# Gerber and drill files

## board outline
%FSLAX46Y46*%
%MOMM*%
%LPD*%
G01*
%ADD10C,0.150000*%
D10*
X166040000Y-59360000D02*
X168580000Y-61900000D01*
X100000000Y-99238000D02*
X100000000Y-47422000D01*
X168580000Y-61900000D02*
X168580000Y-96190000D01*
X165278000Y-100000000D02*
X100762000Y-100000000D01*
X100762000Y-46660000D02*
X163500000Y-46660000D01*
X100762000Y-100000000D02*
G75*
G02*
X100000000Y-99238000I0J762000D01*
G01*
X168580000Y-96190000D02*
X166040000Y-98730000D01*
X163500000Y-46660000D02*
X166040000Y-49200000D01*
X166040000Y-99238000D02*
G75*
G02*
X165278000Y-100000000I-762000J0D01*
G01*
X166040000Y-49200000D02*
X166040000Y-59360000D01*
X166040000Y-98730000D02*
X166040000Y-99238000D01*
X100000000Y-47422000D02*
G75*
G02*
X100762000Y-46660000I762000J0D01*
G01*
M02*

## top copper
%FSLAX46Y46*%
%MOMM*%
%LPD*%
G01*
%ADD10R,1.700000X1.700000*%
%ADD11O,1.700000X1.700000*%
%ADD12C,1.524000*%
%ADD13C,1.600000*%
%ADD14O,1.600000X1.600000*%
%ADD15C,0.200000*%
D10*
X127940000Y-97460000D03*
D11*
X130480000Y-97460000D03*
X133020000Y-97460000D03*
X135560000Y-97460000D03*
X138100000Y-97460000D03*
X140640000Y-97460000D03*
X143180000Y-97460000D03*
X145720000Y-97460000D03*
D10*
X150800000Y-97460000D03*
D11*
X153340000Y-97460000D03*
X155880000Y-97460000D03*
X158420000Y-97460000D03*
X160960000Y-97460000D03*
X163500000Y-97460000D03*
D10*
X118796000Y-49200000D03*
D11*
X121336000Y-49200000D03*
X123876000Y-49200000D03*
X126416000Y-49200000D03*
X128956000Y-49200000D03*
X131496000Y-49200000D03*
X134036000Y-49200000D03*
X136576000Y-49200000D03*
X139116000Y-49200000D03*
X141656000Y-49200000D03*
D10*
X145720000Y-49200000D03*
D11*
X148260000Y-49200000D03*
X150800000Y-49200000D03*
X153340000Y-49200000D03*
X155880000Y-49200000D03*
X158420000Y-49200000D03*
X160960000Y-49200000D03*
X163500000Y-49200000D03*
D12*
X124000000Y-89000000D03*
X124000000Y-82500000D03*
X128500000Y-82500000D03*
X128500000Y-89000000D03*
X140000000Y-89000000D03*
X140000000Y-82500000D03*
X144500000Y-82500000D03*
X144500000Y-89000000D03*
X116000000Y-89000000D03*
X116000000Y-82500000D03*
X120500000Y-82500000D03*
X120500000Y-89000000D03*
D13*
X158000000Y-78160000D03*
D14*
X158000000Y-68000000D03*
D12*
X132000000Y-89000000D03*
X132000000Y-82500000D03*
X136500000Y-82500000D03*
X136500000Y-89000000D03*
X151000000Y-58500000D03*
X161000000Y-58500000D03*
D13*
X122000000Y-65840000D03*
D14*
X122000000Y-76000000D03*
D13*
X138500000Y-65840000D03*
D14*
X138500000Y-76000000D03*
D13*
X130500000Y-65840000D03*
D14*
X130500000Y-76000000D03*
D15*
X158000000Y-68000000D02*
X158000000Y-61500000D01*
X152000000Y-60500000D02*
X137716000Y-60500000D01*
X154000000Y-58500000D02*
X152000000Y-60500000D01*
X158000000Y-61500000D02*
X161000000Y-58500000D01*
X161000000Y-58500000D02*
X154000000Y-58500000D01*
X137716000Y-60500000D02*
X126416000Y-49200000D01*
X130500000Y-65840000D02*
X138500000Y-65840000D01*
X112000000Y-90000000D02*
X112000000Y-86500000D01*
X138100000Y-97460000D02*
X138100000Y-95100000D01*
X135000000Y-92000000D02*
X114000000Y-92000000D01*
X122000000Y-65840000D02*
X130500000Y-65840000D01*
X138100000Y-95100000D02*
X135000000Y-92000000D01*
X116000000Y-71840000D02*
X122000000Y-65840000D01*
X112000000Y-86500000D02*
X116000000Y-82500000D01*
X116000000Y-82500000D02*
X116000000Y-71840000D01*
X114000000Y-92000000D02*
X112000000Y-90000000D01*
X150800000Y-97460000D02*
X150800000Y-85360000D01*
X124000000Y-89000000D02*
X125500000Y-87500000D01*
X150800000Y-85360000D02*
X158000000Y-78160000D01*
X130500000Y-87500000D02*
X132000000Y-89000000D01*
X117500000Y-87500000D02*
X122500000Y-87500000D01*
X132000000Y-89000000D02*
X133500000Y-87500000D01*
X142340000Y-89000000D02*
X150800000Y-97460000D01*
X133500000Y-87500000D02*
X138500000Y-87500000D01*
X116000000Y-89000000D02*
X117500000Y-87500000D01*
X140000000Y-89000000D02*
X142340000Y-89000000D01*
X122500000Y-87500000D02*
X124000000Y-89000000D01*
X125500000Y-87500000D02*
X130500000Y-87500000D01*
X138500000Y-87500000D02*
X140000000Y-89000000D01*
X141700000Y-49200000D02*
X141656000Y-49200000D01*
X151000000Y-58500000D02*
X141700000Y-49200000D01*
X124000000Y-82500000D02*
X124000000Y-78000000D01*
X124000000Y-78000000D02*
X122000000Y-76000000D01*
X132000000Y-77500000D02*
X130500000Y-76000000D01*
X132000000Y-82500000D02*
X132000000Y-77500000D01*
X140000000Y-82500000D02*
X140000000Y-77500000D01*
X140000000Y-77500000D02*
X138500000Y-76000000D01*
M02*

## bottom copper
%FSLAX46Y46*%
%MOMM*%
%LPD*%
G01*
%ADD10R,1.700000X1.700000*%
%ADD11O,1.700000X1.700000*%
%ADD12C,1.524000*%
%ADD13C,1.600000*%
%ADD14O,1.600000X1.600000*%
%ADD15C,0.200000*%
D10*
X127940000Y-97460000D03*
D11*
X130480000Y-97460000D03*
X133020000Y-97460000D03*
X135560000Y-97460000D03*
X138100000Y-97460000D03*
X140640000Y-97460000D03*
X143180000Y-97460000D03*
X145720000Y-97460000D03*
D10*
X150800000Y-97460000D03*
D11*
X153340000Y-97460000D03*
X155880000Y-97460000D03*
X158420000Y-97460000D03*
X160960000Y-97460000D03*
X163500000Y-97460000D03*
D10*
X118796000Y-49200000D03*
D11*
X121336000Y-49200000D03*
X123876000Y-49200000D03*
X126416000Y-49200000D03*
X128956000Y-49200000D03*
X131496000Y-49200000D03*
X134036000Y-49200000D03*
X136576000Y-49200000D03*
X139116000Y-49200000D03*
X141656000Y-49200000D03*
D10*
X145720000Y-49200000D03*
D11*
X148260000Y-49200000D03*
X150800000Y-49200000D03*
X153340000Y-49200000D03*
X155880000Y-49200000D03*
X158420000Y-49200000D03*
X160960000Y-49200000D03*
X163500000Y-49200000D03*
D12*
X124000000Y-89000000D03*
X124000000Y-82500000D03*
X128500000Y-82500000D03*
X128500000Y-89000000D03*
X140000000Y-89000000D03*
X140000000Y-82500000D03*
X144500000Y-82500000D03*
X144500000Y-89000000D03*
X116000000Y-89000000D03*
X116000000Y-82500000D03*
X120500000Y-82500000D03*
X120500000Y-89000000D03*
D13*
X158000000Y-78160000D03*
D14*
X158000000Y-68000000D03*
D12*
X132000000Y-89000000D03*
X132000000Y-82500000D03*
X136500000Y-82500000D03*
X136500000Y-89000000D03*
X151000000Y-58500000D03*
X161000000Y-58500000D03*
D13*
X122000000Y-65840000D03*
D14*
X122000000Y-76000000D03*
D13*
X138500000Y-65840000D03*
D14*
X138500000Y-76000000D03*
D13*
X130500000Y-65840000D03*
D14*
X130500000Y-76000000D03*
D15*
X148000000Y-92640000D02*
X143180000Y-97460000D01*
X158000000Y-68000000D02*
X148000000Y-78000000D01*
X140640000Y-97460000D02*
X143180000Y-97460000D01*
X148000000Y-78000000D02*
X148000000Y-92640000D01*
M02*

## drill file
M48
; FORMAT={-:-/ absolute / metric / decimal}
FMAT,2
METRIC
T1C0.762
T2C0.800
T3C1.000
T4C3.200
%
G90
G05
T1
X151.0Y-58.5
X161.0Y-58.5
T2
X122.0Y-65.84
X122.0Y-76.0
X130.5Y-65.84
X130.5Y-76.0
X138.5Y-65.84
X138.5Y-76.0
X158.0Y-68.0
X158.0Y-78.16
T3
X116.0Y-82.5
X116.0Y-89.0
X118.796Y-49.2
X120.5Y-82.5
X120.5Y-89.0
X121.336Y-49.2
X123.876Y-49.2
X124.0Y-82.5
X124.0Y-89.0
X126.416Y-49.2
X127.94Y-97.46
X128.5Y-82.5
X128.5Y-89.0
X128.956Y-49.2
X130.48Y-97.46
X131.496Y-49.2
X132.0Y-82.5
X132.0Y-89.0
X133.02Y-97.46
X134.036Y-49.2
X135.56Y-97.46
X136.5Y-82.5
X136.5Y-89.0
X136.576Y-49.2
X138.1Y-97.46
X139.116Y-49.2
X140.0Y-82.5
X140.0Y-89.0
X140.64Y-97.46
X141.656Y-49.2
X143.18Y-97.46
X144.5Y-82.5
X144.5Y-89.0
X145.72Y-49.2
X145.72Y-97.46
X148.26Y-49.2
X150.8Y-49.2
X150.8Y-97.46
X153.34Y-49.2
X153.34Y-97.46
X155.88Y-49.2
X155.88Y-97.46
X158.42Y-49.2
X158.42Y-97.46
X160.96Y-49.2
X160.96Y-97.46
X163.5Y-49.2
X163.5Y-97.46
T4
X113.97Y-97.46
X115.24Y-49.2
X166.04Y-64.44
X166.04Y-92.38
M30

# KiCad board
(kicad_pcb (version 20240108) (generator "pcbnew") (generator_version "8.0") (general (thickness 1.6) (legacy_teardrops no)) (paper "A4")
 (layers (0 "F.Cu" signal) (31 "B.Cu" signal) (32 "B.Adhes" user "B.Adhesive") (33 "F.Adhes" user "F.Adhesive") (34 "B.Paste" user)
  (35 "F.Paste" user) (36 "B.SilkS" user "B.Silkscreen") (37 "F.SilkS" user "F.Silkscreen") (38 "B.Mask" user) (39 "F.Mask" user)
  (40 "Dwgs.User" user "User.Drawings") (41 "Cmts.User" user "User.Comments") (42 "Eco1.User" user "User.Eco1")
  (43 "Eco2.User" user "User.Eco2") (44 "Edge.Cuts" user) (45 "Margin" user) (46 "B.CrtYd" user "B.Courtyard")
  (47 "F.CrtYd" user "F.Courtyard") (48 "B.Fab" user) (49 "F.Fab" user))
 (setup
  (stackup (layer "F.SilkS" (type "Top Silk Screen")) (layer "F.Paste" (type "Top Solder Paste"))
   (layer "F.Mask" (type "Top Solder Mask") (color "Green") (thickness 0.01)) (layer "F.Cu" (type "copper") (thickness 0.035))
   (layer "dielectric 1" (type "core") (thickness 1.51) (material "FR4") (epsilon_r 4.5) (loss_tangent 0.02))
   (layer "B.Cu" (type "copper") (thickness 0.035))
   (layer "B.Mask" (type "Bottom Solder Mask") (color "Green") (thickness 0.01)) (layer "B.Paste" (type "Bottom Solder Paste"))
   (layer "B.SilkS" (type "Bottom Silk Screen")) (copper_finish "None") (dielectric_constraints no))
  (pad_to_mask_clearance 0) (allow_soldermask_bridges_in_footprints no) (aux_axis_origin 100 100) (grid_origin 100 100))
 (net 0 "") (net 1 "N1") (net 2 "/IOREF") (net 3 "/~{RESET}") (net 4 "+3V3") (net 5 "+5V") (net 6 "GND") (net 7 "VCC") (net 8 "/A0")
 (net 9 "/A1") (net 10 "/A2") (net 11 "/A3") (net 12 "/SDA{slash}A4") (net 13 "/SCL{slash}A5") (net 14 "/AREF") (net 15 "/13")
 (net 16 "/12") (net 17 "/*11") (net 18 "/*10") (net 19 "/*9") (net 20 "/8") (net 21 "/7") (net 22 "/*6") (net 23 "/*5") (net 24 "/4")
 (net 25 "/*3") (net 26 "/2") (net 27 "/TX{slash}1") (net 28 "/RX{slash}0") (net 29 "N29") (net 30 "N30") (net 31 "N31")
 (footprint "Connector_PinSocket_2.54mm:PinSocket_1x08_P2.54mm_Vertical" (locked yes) (layer "F.Cu") (at 127.94 97.46 90)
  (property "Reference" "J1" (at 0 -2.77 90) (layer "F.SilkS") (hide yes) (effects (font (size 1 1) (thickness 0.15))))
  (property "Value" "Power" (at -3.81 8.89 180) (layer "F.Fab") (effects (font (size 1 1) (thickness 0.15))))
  (pad "1" thru_hole rect (at 0 0 90) (size 1.7 1.7) (drill 1) (layers "*.Cu" "*.Mask") (remove_unused_layers no) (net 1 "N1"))
  (pad "2" thru_hole oval (at 0 2.54 90) (size 1.7 1.7) (drill 1) (layers "*.Cu" "*.Mask") (remove_unused_layers no) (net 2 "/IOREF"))
  (pad "3" thru_hole oval (at 0 5.08 90) (size 1.7 1.7) (drill 1) (layers "*.Cu" "*.Mask") (remove_unused_layers no) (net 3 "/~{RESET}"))
  (pad "4" thru_hole oval (at 0 7.62 90) (size 1.7 1.7) (drill 1) (layers "*.Cu" "*.Mask") (remove_unused_layers no) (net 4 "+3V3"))
  (pad "5" thru_hole oval (at 0 10.16 90) (size 1.7 1.7) (drill 1) (layers "*.Cu" "*.Mask") (remove_unused_layers no) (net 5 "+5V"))
  (pad "6" thru_hole oval (at 0 12.7 90) (size 1.7 1.7) (drill 1) (layers "*.Cu" "*.Mask") (remove_unused_layers no) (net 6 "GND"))
  (pad "7" thru_hole oval (at 0 15.24 90) (size 1.7 1.7) (drill 1) (layers "*.Cu" "*.Mask") (remove_unused_layers no) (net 6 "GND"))
  (pad "8" thru_hole oval (at 0 17.78 90) (size 1.7 1.7) (drill 1) (layers "*.Cu" "*.Mask") (remove_unused_layers no) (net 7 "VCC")))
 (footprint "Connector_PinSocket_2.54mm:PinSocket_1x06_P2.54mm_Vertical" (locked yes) (layer "F.Cu") (at 150.8 97.46 90)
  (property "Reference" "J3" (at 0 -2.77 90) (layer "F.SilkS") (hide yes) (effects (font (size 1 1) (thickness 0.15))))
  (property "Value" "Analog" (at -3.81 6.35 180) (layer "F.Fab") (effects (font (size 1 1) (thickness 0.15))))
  (pad "1" thru_hole rect (at 0 0 90) (size 1.7 1.7) (drill 1) (layers "*.Cu" "*.Mask") (remove_unused_layers no) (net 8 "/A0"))
  (pad "2" thru_hole oval (at 0 2.54 90) (size 1.7 1.7) (drill 1) (layers "*.Cu" "*.Mask") (remove_unused_layers no) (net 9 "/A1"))
  (pad "3" thru_hole oval (at 0 5.08 90) (size 1.7 1.7) (drill 1) (layers "*.Cu" "*.Mask") (remove_unused_layers no) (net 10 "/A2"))
  (pad "4" thru_hole oval (at 0 7.62 90) (size 1.7 1.7) (drill 1) (layers "*.Cu" "*.Mask") (remove_unused_layers no) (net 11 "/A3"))
  (pad "5" thru_hole oval (at 0 10.16 90) (size 1.7 1.7) (drill 1) (layers "*.Cu" "*.Mask") (remove_unused_layers no)
   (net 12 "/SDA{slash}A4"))
  (pad "6" thru_hole oval (at 0 12.7 90) (size 1.7 1.7) (drill 1) (layers "*.Cu" "*.Mask") (remove_unused_layers no)
   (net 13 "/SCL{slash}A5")))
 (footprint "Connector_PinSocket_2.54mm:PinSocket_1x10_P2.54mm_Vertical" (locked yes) (layer "F.Cu") (at 118.796 49.2 90)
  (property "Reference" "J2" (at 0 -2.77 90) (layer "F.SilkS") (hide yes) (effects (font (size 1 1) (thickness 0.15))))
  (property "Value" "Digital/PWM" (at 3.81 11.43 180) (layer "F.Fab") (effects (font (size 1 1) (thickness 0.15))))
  (pad "1" thru_hole rect (at 0 0 90) (size 1.7 1.7) (drill 1) (layers "*.Cu" "*.Mask") (remove_unused_layers no) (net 13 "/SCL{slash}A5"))
  (pad "2" thru_hole oval (at 0 2.54 90) (size 1.7 1.7) (drill 1) (layers "*.Cu" "*.Mask") (remove_unused_layers no)
   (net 12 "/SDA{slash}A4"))
  (pad "3" thru_hole oval (at 0 5.08 90) (size 1.7 1.7) (drill 1) (layers "*.Cu" "*.Mask") (remove_unused_layers no) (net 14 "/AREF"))
  (pad "4" thru_hole oval (at 0 7.62 90) (size 1.7 1.7) (drill 1) (layers "*.Cu" "*.Mask") (remove_unused_layers no) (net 6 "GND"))
  (pad "5" thru_hole oval (at 0 10.16 90) (size 1.7 1.7) (drill 1) (layers "*.Cu" "*.Mask") (remove_unused_layers no) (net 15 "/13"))
  (pad "6" thru_hole oval (at 0 12.7 90) (size 1.7 1.7) (drill 1) (layers "*.Cu" "*.Mask") (remove_unused_layers no) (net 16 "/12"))
  (pad "7" thru_hole oval (at 0 15.24 90) (size 1.7 1.7) (drill 1) (layers "*.Cu" "*.Mask") (remove_unused_layers no) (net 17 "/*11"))
  (pad "8" thru_hole oval (at 0 17.78 90) (size 1.7 1.7) (drill 1) (layers "*.Cu" "*.Mask") (remove_unused_layers no) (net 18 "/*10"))
  (pad "9" thru_hole oval (at 0 20.32 90) (size 1.7 1.7) (drill 1) (layers "*.Cu" "*.Mask") (remove_unused_layers no) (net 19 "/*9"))
  (pad "10" thru_hole oval (at 0 22.86 90) (size 1.7 1.7) (drill 1) (layers "*.Cu" "*.Mask") (remove_unused_layers no) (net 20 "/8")))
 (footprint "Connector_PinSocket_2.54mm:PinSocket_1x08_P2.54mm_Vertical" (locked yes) (layer "F.Cu") (at 145.72 49.2 90)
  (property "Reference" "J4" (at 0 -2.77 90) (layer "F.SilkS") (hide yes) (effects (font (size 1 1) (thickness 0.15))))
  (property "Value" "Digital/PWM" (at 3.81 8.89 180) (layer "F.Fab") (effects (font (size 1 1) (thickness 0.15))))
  (pad "1" thru_hole rect (at 0 0 90) (size 1.7 1.7) (drill 1) (layers "*.Cu" "*.Mask") (remove_unused_layers no) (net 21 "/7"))
  (pad "2" thru_hole oval (at 0 2.54 90) (size 1.7 1.7) (drill 1) (layers "*.Cu" "*.Mask") (remove_unused_layers no) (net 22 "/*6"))
  (pad "3" thru_hole oval (at 0 5.08 90) (size 1.7 1.7) (drill 1) (layers "*.Cu" "*.Mask") (remove_unused_layers no) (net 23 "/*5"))
  (pad "4" thru_hole oval (at 0 7.62 90) (size 1.7 1.7) (drill 1) (layers "*.Cu" "*.Mask") (remove_unused_layers no) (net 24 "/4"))
  (pad "5" thru_hole oval (at 0 10.16 90) (size 1.7 1.7) (drill 1) (layers "*.Cu" "*.Mask") (remove_unused_layers no) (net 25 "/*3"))
  (pad "6" thru_hole oval (at 0 12.7 90) (size 1.7 1.7) (drill 1) (layers "*.Cu" "*.Mask") (remove_unused_layers no) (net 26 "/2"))
  (pad "7" thru_hole oval (at 0 15.24 90) (size 1.7 1.7) (drill 1) (layers "*.Cu" "*.Mask") (remove_unused_layers no) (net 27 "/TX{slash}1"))
  (pad "8" thru_hole oval (at 0 17.78 90) (size 1.7 1.7) (drill 1) (layers "*.Cu" "*.Mask") (remove_unused_layers no) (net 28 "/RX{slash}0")))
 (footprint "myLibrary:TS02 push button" (layer "F.Cu") (at 124 89 90)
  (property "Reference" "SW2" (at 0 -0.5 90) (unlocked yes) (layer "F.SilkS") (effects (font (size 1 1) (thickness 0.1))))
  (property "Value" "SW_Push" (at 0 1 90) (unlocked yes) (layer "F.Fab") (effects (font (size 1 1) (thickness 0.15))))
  (pad "1" thru_hole circle (at 0 0 90) (size 1.524 1.524) (drill 1) (layers "*.Cu" "*.Mask") (remove_unused_layers no) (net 8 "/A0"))
  (pad "2" thru_hole circle (at 6.5 0 90) (size 1.524 1.524) (drill 1) (layers "*.Cu" "*.Mask") (remove_unused_layers no) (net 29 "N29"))
  (pad "3" thru_hole circle (at 6.5 4.5 90) (size 1.524 1.524) (drill 1) (layers "*.Cu" "*.Mask") (remove_unused_layers no))
  (pad "4" thru_hole circle (at 0 4.5 90) (size 1.524 1.524) (drill 1) (layers "*.Cu" "*.Mask") (remove_unused_layers no)))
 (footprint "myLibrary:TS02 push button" (layer "F.Cu") (at 140 89 90)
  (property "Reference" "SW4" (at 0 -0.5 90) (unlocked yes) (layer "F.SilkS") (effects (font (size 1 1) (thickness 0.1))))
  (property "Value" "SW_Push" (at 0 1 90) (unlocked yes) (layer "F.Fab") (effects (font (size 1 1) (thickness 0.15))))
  (pad "1" thru_hole circle (at 0 0 90) (size 1.524 1.524) (drill 1) (layers "*.Cu" "*.Mask") (remove_unused_layers no) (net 8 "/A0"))
  (pad "2" thru_hole circle (at 6.5 0 90) (size 1.524 1.524) (drill 1) (layers "*.Cu" "*.Mask") (remove_unused_layers no) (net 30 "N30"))
  (pad "3" thru_hole circle (at 6.5 4.5 90) (size 1.524 1.524) (drill 1) (layers "*.Cu" "*.Mask") (remove_unused_layers no))
  (pad "4" thru_hole circle (at 0 4.5 90) (size 1.524 1.524) (drill 1) (layers "*.Cu" "*.Mask") (remove_unused_layers no)))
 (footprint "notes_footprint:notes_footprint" (layer "F.Cu") (at 123.5 57.5)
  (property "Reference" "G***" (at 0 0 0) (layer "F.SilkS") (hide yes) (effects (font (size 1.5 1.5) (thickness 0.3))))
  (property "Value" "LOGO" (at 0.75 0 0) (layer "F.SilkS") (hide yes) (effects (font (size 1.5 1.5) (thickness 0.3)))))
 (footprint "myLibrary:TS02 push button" (layer "F.Cu") (at 116 89 90)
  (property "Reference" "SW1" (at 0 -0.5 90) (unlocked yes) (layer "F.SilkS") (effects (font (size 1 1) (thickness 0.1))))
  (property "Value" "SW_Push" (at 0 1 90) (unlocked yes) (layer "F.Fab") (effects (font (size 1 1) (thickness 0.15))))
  (pad "1" thru_hole circle (at 0 0 90) (size 1.524 1.524) (drill 1) (layers "*.Cu" "*.Mask") (remove_unused_layers no) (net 8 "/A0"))
  (pad "2" thru_hole circle (at 6.5 0 90) (size 1.524 1.524) (drill 1) (layers "*.Cu" "*.Mask") (remove_unused_layers no) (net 5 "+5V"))
  (pad "3" thru_hole circle (at 6.5 4.5 90) (size 1.524 1.524) (drill 1) (layers "*.Cu" "*.Mask") (remove_unused_layers no))
  (pad "4" thru_hole circle (at 0 4.5 90) (size 1.524 1.524) (drill 1) (layers "*.Cu" "*.Mask") (remove_unused_layers no)))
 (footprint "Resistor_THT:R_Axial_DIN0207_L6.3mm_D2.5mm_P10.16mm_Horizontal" (layer "F.Cu") (at 158 78.16 90)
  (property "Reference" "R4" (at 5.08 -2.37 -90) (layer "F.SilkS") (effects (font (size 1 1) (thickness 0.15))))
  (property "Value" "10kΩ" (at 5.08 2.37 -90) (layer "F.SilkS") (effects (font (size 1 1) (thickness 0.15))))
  (pad "1" thru_hole circle (at 0 0 90) (size 1.6 1.6) (drill 0.8) (layers "*.Cu" "*.Mask") (remove_unused_layers no) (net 8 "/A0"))
  (pad "2" thru_hole oval (at 10.16 0 90) (size 1.6 1.6) (drill 0.8) (layers "*.Cu" "*.Mask") (remove_unused_layers no) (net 6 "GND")))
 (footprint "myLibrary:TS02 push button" (layer "F.Cu") (at 132 89 90)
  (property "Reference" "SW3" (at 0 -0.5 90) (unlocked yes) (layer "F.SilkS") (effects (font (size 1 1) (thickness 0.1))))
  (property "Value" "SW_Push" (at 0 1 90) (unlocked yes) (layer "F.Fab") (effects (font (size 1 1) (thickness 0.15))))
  (pad "1" thru_hole circle (at 0 0 90) (size 1.524 1.524) (drill 1) (layers "*.Cu" "*.Mask") (remove_unused_layers no) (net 8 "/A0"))
  (pad "2" thru_hole circle (at 6.5 0 90) (size 1.524 1.524) (drill 1) (layers "*.Cu" "*.Mask") (remove_unused_layers no) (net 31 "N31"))
  (pad "3" thru_hole circle (at 6.5 4.5 90) (size 1.524 1.524) (drill 1) (layers "*.Cu" "*.Mask") (remove_unused_layers no))
  (pad "4" thru_hole circle (at 0 4.5 90) (size 1.524 1.524) (drill 1) (layers "*.Cu" "*.Mask") (remove_unused_layers no)))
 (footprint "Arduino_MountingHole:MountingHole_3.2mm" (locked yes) (layer "F.Cu") (at 115.24 49.2)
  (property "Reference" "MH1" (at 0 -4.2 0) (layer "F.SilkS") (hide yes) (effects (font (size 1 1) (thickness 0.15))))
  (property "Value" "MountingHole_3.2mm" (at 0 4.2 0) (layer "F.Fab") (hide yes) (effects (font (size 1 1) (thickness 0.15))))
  (pad "" np_thru_hole circle (at 0 0) (size 3.2 3.2) (drill 3.2) (layers "*.Cu" "*.Mask")))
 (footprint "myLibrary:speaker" (layer "F.Cu") (at 156 58.5)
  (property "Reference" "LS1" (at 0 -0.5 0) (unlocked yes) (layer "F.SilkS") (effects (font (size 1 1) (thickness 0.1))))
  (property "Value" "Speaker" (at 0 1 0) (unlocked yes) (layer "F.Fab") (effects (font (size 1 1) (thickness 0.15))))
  (pad "1" thru_hole circle (at -5 0) (size 1.524 1.524) (drill 0.762) (layers "*.Cu" "*.Mask") (remove_unused_layers no) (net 20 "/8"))
  (pad "2" thru_hole circle (at 5 0) (size 1.524 1.524) (drill 0.762) (layers "*.Cu" "*.Mask") (remove_unused_layers no) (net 6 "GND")))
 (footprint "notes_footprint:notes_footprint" (layer "F.Cu") (at 115.5 54.5)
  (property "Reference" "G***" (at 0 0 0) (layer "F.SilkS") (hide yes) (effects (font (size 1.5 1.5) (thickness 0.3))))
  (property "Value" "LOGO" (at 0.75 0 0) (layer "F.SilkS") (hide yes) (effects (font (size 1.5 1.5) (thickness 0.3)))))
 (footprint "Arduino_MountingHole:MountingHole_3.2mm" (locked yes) (layer "F.Cu") (at 113.97 97.46)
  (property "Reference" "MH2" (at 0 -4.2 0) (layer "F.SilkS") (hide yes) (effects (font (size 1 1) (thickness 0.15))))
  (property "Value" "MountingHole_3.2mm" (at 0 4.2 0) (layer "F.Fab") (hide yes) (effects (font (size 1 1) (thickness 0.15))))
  (pad "" np_thru_hole circle (at 0 0) (size 3.2 3.2) (drill 3.2) (layers "*.Cu" "*.Mask")))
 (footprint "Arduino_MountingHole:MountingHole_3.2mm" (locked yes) (layer "F.Cu") (at 166.04 64.44)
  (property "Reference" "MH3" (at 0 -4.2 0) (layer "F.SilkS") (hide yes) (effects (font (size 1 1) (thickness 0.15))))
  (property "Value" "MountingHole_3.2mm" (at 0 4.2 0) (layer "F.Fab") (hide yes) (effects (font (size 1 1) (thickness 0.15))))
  (pad "" np_thru_hole circle (at 0 0) (size 3.2 3.2) (drill 3.2) (layers "*.Cu" "*.Mask")))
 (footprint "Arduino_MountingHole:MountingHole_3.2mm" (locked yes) (layer "F.Cu") (at 166.04 92.38)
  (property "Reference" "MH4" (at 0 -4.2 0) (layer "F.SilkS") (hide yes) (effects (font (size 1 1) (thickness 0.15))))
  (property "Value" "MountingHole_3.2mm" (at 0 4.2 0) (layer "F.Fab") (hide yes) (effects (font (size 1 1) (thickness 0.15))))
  (pad "" np_thru_hole circle (at 0 0) (size 3.2 3.2) (drill 3.2) (layers "*.Cu" "*.Mask")))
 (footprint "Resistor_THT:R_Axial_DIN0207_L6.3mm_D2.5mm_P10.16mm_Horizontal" (layer "B.Cu") (at 122 65.84 -90)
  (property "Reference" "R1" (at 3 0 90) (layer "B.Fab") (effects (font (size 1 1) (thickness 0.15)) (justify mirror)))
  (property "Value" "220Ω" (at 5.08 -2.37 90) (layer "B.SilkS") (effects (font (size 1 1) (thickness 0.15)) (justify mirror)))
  (pad "1" thru_hole circle (at 0 0 270) (size 1.6 1.6) (drill 0.8) (layers "*.Cu" "*.Mask") (remove_unused_layers no) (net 5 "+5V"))
  (pad "2" thru_hole oval (at 10.16 0 270) (size 1.6 1.6) (drill 0.8) (layers "*.Cu" "*.Mask") (remove_unused_layers no) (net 29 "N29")))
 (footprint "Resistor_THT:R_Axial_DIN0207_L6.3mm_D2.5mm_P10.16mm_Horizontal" (layer "B.Cu") (at 138.5 65.84 -90)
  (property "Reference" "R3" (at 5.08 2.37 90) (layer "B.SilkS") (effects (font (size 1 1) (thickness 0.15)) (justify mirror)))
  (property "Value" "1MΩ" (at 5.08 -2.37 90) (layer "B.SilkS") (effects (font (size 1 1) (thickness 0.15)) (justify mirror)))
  (pad "1" thru_hole circle (at 0 0 270) (size 1.6 1.6) (drill 0.8) (layers "*.Cu" "*.Mask") (remove_unused_layers no) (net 5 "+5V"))
  (pad "2" thru_hole oval (at 10.16 0 270) (size 1.6 1.6) (drill 0.8) (layers "*.Cu" "*.Mask") (remove_unused_layers no) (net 30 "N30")))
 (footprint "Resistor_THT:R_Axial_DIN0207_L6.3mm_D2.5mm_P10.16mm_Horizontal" (layer "B.Cu") (at 130.5 65.84 -90)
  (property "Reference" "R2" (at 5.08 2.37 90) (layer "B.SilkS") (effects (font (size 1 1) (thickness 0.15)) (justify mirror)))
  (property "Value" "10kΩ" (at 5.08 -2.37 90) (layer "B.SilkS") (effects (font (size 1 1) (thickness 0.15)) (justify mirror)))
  (pad "1" thru_hole circle (at 0 0 270) (size 1.6 1.6) (drill 0.8) (layers "*.Cu" "*.Mask") (remove_unused_layers no) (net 5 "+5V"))
  (pad "2" thru_hole oval (at 10.16 0 270) (size 1.6 1.6) (drill 0.8) (layers "*.Cu" "*.Mask") (remove_unused_layers no) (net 31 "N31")))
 (gr_line (start 166.04 59.36) (end 168.58 61.9) (stroke (width 0.15) (type solid)) (layer "Edge.Cuts"))
 (gr_line (start 100 99.238) (end 100 47.422) (stroke (width 0.15) (type solid)) (layer "Edge.Cuts"))
 (gr_line (start 168.58 61.9) (end 168.58 96.19) (stroke (width 0.15) (type solid)) (layer "Edge.Cuts"))
 (gr_line (start 165.278 100) (end 100.762 100) (stroke (width 0.15) (type solid)) (layer "Edge.Cuts"))
 (gr_line (start 100.762 46.66) (end 163.5 46.66) (stroke (width 0.15) (type solid)) (layer "Edge.Cuts"))
 (gr_arc (start 100.762 100) (mid 100.223185 99.776815) (end 100 99.238) (stroke (width 0.15) (type solid)) (layer "Edge.Cuts"))
 (gr_line (start 168.58 96.19) (end 166.04 98.73) (stroke (width 0.15) (type solid)) (layer "Edge.Cuts"))
 (gr_line (start 163.5 46.66) (end 166.04 49.2) (stroke (width 0.15) (type solid)) (layer "Edge.Cuts"))
 (gr_arc (start 166.04 99.238) (mid 165.816815 99.776815) (end 165.278 100) (stroke (width 0.15) (type solid)) (layer "Edge.Cuts"))
 (gr_line (start 166.04 49.2) (end 166.04 59.36) (stroke (width 0.15) (type solid)) (layer "Edge.Cuts"))
 (gr_line (start 166.04 98.73) (end 166.04 99.238) (stroke (width 0.15) (type solid)) (layer "Edge.Cuts"))
 (gr_arc (start 100 47.422) (mid 100.223185 46.883185) (end 100.762 46.66) (stroke (width 0.15) (type solid)) (layer "Edge.Cuts"))
 (segment (start 158 68) (end 158 61.5) (width 0.2) (layer "F.Cu") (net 6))
 (segment (start 152 60.5) (end 137.716 60.5) (width 0.2) (layer "F.Cu") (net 6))
 (segment (start 154 58.5) (end 152 60.5) (width 0.2) (layer "F.Cu") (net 6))
 (segment (start 158 61.5) (end 161 58.5) (width 0.2) (layer "F.Cu") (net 6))
 (segment (start 161 58.5) (end 154 58.5) (width 0.2) (layer "F.Cu") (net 6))
 (segment (start 137.716 60.5) (end 126.416 49.2) (width 0.2) (layer "F.Cu") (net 6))
 (segment (start 148 92.64) (end 143.18 97.46) (width 0.2) (layer "B.Cu") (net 6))
 (segment (start 158 68) (end 148 78) (width 0.2) (layer "B.Cu") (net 6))
 (segment (start 140.64 97.46) (end 143.18 97.46) (width 0.2) (layer "B.Cu") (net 6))
 (segment (start 148 78) (end 148 92.64) (width 0.2) (layer "B.Cu") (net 6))
 (segment (start 130.5 65.84) (end 138.5 65.84) (width 0.2) (layer "F.Cu") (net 5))
 (segment (start 112 90) (end 112 86.5) (width 0.2) (layer "F.Cu") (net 5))
 (segment (start 138.1 97.46) (end 138.1 95.1) (width 0.2) (layer "F.Cu") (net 5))
 (segment (start 135 92) (end 114 92) (width 0.2) (layer "F.Cu") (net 5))
 (segment (start 122 65.84) (end 130.5 65.84) (width 0.2) (layer "F.Cu") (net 5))
 (segment (start 138.1 95.1) (end 135 92) (width 0.2) (layer "F.Cu") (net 5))
 (segment (start 116 71.84) (end 122 65.84) (width 0.2) (layer "F.Cu") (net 5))
 (segment (start 112 86.5) (end 116 82.5) (width 0.2) (layer "F.Cu") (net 5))
 (segment (start 116 82.5) (end 116 71.84) (width 0.2) (layer "F.Cu") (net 5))
 (segment (start 114 92) (end 112 90) (width 0.2) (layer "F.Cu") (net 5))
 (segment (start 150.8 97.46) (end 150.8 85.36) (width 0.2) (layer "F.Cu") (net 8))
 (segment (start 124 89) (end 125.5 87.5) (width 0.2) (layer "F.Cu") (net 8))
 (segment (start 150.8 85.36) (end 158 78.16) (width 0.2) (layer "F.Cu") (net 8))
 (segment (start 130.5 87.5) (end 132 89) (width 0.2) (layer "F.Cu") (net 8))
 (segment (start 117.5 87.5) (end 122.5 87.5) (width 0.2) (layer "F.Cu") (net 8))
 (segment (start 132 89) (end 133.5 87.5) (width 0.2) (layer "F.Cu") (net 8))
 (segment (start 142.34 89) (end 150.8 97.46) (width 0.2) (layer "F.Cu") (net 8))
 (segment (start 133.5 87.5) (end 138.5 87.5) (width 0.2) (layer "F.Cu") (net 8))
 (segment (start 116 89) (end 117.5 87.5) (width 0.2) (layer "F.Cu") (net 8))
 (segment (start 140 89) (end 142.34 89) (width 0.2) (layer "F.Cu") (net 8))
 (segment (start 122.5 87.5) (end 124 89) (width 0.2) (layer "F.Cu") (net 8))
 (segment (start 125.5 87.5) (end 130.5 87.5) (width 0.2) (layer "F.Cu") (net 8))
 (segment (start 138.5 87.5) (end 140 89) (width 0.2) (layer "F.Cu") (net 8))
 (segment (start 141.7 49.2) (end 141.656 49.2) (width 0.2) (layer "F.Cu") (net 20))
 (segment (start 151 58.5) (end 141.7 49.2) (width 0.2) (layer "F.Cu") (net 20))
 (segment (start 124 82.5) (end 124 78) (width 0.2) (layer "F.Cu") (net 29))
 (segment (start 124 78) (end 122 76) (width 0.2) (layer "F.Cu") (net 29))
 (segment (start 132 77.5) (end 130.5 76) (width 0.2) (layer "F.Cu") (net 31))
 (segment (start 132 82.5) (end 132 77.5) (width 0.2) (layer "F.Cu") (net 31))
 (segment (start 140 82.5) (end 140 77.5) (width 0.2) (layer "F.Cu") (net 30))
 (segment (start 140 77.5) (end 138.5 76) (width 0.2) (layer "F.Cu") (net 30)))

